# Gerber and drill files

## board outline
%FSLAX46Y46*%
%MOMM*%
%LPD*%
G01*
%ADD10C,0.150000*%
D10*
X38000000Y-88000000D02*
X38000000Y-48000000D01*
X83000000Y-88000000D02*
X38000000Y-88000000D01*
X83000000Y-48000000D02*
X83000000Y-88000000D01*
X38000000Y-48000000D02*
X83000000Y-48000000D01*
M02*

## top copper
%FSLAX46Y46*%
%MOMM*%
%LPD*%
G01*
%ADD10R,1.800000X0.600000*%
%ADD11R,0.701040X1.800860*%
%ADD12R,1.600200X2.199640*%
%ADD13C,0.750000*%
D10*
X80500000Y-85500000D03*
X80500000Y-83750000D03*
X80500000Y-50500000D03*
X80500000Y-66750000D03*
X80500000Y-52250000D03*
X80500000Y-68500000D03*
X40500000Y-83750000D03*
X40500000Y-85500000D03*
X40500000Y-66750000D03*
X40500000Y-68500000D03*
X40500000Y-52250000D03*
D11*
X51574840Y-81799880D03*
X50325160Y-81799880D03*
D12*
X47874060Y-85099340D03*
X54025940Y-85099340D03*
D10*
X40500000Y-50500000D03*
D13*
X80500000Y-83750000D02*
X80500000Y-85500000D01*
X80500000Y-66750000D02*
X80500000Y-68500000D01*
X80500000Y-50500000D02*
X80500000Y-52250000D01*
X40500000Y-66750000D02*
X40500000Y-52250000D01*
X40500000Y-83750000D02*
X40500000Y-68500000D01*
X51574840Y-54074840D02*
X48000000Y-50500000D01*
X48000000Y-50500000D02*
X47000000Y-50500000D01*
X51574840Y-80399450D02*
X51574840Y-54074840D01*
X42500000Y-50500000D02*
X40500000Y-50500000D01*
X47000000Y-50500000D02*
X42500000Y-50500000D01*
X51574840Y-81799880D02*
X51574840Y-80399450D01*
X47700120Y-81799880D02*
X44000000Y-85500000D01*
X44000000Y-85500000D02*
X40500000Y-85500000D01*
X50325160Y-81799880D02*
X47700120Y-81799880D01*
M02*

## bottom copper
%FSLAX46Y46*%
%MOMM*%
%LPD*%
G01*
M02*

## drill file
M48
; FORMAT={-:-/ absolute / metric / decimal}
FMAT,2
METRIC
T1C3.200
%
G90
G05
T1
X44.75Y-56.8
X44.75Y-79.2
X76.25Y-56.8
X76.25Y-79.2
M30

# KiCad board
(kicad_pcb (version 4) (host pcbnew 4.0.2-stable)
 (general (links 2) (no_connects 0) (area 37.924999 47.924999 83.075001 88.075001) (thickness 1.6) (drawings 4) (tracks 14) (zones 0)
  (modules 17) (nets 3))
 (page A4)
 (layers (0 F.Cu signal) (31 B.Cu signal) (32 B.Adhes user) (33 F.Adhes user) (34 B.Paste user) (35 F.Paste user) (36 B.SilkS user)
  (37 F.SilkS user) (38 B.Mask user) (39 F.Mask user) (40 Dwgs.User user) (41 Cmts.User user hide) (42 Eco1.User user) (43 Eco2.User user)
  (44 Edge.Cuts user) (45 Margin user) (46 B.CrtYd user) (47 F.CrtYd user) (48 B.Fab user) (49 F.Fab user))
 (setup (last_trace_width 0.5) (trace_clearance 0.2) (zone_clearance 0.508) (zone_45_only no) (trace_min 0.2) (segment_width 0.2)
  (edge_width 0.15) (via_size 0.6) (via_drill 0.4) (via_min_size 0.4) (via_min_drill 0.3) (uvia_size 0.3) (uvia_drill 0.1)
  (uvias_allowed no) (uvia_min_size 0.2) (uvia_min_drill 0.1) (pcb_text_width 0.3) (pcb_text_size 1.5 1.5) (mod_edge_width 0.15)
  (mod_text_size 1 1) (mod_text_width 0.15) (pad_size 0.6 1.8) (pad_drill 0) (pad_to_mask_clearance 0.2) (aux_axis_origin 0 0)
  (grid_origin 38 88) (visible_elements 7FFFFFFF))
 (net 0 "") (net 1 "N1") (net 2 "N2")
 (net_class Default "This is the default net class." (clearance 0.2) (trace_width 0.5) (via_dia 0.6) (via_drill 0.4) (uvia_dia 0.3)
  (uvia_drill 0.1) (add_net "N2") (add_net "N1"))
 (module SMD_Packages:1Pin (layer F.Cu) (at 80.5 85.5 90)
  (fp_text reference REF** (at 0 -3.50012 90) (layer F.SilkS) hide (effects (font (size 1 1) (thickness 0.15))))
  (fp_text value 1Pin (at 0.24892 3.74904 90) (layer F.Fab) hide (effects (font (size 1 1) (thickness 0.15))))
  (pad 1 smd rect (at 0 0 90) (size 0.6 1.8) (layers F.Cu F.Paste F.SilkS F.Mask)))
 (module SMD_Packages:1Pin (layer F.Cu) (at 80.5 83.75 90)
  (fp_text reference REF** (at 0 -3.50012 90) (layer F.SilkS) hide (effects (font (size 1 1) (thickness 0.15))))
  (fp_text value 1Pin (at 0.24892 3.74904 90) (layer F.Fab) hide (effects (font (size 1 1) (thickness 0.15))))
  (pad 1 smd rect (at 0 0 90) (size 0.6 1.8) (layers F.Cu F.Paste F.SilkS F.Mask)))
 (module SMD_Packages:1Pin (layer F.Cu) (at 80.5 50.5 90)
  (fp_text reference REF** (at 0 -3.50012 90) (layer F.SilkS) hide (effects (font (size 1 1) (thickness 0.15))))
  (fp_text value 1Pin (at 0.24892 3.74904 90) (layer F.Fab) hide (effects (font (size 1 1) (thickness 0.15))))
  (pad 1 smd rect (at 0 0 90) (size 0.6 1.8) (layers F.Cu F.Paste F.SilkS F.Mask)))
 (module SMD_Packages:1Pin (layer F.Cu) (at 80.5 66.75 90)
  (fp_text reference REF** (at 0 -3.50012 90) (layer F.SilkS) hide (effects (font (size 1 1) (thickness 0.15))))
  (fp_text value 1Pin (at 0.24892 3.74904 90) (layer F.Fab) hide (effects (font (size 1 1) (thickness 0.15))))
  (pad 1 smd rect (at 0 0 90) (size 0.6 1.8) (layers F.Cu F.Paste F.SilkS F.Mask)))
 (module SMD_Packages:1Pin (layer F.Cu) (at 80.5 52.25 90)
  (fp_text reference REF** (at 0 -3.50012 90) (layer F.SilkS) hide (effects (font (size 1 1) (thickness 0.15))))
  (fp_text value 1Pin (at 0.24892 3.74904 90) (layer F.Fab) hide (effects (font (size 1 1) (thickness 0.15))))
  (pad 1 smd rect (at 0 0 90) (size 0.6 1.8) (layers F.Cu F.Paste F.SilkS F.Mask)))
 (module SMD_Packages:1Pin (layer F.Cu) (at 80.5 68.5 90)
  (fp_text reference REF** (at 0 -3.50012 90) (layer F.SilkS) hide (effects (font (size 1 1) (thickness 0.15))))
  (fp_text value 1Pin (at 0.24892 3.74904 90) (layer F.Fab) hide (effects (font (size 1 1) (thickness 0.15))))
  (pad 1 smd rect (at 0 0 90) (size 0.6 1.8) (layers F.Cu F.Paste F.SilkS F.Mask)))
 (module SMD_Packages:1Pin (layer F.Cu) (at 40.5 83.75 90)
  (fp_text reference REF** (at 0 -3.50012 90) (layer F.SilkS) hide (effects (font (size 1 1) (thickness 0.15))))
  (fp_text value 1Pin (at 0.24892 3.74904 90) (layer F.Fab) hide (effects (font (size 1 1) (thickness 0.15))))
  (pad 1 smd rect (at 0 0 90) (size 0.6 1.8) (layers F.Cu F.Paste F.SilkS F.Mask)))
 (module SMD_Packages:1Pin (layer F.Cu) (at 40.5 85.5 90)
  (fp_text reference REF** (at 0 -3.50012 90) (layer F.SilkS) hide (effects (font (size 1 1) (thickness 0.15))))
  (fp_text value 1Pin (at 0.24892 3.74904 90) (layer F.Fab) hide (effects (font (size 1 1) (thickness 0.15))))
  (pad 1 smd rect (at 0 0 90) (size 0.6 1.8) (layers F.Cu F.Paste F.SilkS F.Mask) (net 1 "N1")))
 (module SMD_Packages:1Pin (layer F.Cu) (at 40.5 66.75 90)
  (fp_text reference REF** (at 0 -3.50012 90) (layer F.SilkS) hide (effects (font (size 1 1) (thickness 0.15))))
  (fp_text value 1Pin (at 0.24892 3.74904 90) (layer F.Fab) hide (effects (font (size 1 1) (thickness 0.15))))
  (pad 1 smd rect (at 0 0 90) (size 0.6 1.8) (layers F.Cu F.Paste F.SilkS F.Mask)))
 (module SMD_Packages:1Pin (layer F.Cu) (at 40.5 68.5 90)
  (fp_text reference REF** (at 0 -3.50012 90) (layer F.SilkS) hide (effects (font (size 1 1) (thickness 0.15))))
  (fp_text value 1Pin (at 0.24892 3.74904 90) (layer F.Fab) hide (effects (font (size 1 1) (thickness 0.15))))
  (pad 1 smd rect (at 0 0 90) (size 0.6 1.8) (layers F.Cu F.Paste F.SilkS F.Mask)))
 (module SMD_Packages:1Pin (layer F.Cu) (at 40.5 52.25 90)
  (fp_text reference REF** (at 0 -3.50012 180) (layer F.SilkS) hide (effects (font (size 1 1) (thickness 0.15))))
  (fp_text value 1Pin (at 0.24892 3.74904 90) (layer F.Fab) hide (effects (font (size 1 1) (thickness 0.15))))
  (pad 1 smd rect (at 0 0 90) (size 0.6 1.8) (layers F.Cu F.Paste F.SilkS F.Mask)))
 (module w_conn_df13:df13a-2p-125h (layer F.Cu) (at 50.95 85.3)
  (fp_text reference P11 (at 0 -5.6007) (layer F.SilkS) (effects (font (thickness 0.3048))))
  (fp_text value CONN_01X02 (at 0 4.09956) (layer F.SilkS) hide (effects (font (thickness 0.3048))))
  (pad 1 smd rect (at 0.62484 -3.50012) (size 0.70104 1.80086) (layers F.Cu F.Paste F.Mask) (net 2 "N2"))
  (pad 2 smd rect (at -0.62484 -3.50012) (size 0.70104 1.80086) (layers F.Cu F.Paste F.Mask) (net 1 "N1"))
  (pad "" smd rect (at -3.07594 -0.20066) (size 1.6002 2.19964) (layers F.Cu F.Paste F.Mask))
  (pad "" smd rect (at 3.07594 -0.20066) (size 1.6002 2.19964) (layers F.Cu F.Paste F.Mask)))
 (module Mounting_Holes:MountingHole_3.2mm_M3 (layer F.Cu) (at 44.75 56.8)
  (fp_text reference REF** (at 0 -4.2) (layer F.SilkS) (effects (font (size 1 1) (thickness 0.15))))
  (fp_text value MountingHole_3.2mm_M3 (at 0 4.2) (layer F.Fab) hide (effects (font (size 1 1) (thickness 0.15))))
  (pad "" np_thru_hole circle (at 0 0) (size 3.2 3.2) (drill 3.2) (layers *.Cu *.Mask F.SilkS)))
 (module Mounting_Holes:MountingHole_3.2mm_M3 (layer F.Cu) (at 76.25 56.8)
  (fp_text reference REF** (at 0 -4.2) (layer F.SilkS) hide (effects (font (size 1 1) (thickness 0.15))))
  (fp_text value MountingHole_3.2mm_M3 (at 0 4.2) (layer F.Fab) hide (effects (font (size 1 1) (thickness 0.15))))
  (pad 1 np_thru_hole circle (at 0 0) (size 3.2 3.2) (drill 3.2) (layers *.Cu *.Mask F.SilkS)))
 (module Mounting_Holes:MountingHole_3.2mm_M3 (layer F.Cu) (at 76.25 79.2)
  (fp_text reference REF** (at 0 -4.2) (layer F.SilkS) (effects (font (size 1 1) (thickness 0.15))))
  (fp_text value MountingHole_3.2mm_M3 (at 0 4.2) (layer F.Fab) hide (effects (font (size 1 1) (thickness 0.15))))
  (pad 1 np_thru_hole circle (at 0 0) (size 3.2 3.2) (drill 3.2) (layers *.Cu *.Mask F.SilkS)))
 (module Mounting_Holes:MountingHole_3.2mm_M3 (layer F.Cu) (at 44.75 79.2)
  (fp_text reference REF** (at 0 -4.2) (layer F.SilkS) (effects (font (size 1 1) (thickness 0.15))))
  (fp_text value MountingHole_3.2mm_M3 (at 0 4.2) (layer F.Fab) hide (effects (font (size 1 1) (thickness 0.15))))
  (pad 1 np_thru_hole circle (at 0 0) (size 3.2 3.2) (drill 3.2) (layers *.Cu *.Mask F.SilkS)))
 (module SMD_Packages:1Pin (layer F.Cu) (at 40.5 50.5 90)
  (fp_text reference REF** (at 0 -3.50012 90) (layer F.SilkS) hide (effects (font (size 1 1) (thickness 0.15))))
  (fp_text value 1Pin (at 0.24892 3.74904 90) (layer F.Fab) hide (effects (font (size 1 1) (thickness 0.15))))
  (pad 1 smd rect (at 0 0 90) (size 0.6 1.8) (layers F.Cu F.Paste F.SilkS F.Mask) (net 2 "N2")))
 (gr_line (start 38 88) (end 38 48) (angle 90) (layer Edge.Cuts) (width 0.15))
 (gr_line (start 83 88) (end 38 88) (angle 90) (layer Edge.Cuts) (width 0.15))
 (gr_line (start 83 48) (end 83 88) (angle 90) (layer Edge.Cuts) (width 0.15))
 (gr_line (start 38 48) (end 83 48) (angle 90) (layer Edge.Cuts) (width 0.15))
 (segment (start 80.5 83.75) (end 80.5 85.5) (width 0.75) (layer F.Cu) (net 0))
 (segment (start 80.5 66.75) (end 80.5 68.5) (width 0.75) (layer F.Cu) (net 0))
 (segment (start 80.5 50.5) (end 80.5 52.25) (width 0.75) (layer F.Cu) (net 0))
 (segment (start 40.5 66.75) (end 40.5 52.25) (width 0.75) (layer F.Cu) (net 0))
 (segment (start 40.5 83.75) (end 40.5 68.5) (width 0.75) (layer F.Cu) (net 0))
 (segment (start 51.57484 54.07484) (end 48 50.5) (width 0.75) (layer F.Cu) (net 2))
 (segment (start 48 50.5) (end 47 50.5) (width 0.75) (layer F.Cu) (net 2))
 (segment (start 51.57484 80.39945) (end 51.57484 54.07484) (width 0.75) (layer F.Cu) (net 2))
 (segment (start 42.5 50.5) (end 40.5 50.5) (width 0.75) (layer F.Cu) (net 2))
 (segment (start 47 50.5) (end 42.5 50.5) (width 0.75) (layer F.Cu) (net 2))
 (segment (start 51.57484 81.79988) (end 51.57484 80.39945) (width 0.75) (layer F.Cu) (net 2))
 (segment (start 47.70012 81.79988) (end 44 85.5) (width 0.75) (layer F.Cu) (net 1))
 (segment (start 44 85.5) (end 40.5 85.5) (width 0.75) (layer F.Cu) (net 1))
 (segment (start 50.32516 81.79988) (end 47.70012 81.79988) (width 0.75) (layer F.Cu) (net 1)))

